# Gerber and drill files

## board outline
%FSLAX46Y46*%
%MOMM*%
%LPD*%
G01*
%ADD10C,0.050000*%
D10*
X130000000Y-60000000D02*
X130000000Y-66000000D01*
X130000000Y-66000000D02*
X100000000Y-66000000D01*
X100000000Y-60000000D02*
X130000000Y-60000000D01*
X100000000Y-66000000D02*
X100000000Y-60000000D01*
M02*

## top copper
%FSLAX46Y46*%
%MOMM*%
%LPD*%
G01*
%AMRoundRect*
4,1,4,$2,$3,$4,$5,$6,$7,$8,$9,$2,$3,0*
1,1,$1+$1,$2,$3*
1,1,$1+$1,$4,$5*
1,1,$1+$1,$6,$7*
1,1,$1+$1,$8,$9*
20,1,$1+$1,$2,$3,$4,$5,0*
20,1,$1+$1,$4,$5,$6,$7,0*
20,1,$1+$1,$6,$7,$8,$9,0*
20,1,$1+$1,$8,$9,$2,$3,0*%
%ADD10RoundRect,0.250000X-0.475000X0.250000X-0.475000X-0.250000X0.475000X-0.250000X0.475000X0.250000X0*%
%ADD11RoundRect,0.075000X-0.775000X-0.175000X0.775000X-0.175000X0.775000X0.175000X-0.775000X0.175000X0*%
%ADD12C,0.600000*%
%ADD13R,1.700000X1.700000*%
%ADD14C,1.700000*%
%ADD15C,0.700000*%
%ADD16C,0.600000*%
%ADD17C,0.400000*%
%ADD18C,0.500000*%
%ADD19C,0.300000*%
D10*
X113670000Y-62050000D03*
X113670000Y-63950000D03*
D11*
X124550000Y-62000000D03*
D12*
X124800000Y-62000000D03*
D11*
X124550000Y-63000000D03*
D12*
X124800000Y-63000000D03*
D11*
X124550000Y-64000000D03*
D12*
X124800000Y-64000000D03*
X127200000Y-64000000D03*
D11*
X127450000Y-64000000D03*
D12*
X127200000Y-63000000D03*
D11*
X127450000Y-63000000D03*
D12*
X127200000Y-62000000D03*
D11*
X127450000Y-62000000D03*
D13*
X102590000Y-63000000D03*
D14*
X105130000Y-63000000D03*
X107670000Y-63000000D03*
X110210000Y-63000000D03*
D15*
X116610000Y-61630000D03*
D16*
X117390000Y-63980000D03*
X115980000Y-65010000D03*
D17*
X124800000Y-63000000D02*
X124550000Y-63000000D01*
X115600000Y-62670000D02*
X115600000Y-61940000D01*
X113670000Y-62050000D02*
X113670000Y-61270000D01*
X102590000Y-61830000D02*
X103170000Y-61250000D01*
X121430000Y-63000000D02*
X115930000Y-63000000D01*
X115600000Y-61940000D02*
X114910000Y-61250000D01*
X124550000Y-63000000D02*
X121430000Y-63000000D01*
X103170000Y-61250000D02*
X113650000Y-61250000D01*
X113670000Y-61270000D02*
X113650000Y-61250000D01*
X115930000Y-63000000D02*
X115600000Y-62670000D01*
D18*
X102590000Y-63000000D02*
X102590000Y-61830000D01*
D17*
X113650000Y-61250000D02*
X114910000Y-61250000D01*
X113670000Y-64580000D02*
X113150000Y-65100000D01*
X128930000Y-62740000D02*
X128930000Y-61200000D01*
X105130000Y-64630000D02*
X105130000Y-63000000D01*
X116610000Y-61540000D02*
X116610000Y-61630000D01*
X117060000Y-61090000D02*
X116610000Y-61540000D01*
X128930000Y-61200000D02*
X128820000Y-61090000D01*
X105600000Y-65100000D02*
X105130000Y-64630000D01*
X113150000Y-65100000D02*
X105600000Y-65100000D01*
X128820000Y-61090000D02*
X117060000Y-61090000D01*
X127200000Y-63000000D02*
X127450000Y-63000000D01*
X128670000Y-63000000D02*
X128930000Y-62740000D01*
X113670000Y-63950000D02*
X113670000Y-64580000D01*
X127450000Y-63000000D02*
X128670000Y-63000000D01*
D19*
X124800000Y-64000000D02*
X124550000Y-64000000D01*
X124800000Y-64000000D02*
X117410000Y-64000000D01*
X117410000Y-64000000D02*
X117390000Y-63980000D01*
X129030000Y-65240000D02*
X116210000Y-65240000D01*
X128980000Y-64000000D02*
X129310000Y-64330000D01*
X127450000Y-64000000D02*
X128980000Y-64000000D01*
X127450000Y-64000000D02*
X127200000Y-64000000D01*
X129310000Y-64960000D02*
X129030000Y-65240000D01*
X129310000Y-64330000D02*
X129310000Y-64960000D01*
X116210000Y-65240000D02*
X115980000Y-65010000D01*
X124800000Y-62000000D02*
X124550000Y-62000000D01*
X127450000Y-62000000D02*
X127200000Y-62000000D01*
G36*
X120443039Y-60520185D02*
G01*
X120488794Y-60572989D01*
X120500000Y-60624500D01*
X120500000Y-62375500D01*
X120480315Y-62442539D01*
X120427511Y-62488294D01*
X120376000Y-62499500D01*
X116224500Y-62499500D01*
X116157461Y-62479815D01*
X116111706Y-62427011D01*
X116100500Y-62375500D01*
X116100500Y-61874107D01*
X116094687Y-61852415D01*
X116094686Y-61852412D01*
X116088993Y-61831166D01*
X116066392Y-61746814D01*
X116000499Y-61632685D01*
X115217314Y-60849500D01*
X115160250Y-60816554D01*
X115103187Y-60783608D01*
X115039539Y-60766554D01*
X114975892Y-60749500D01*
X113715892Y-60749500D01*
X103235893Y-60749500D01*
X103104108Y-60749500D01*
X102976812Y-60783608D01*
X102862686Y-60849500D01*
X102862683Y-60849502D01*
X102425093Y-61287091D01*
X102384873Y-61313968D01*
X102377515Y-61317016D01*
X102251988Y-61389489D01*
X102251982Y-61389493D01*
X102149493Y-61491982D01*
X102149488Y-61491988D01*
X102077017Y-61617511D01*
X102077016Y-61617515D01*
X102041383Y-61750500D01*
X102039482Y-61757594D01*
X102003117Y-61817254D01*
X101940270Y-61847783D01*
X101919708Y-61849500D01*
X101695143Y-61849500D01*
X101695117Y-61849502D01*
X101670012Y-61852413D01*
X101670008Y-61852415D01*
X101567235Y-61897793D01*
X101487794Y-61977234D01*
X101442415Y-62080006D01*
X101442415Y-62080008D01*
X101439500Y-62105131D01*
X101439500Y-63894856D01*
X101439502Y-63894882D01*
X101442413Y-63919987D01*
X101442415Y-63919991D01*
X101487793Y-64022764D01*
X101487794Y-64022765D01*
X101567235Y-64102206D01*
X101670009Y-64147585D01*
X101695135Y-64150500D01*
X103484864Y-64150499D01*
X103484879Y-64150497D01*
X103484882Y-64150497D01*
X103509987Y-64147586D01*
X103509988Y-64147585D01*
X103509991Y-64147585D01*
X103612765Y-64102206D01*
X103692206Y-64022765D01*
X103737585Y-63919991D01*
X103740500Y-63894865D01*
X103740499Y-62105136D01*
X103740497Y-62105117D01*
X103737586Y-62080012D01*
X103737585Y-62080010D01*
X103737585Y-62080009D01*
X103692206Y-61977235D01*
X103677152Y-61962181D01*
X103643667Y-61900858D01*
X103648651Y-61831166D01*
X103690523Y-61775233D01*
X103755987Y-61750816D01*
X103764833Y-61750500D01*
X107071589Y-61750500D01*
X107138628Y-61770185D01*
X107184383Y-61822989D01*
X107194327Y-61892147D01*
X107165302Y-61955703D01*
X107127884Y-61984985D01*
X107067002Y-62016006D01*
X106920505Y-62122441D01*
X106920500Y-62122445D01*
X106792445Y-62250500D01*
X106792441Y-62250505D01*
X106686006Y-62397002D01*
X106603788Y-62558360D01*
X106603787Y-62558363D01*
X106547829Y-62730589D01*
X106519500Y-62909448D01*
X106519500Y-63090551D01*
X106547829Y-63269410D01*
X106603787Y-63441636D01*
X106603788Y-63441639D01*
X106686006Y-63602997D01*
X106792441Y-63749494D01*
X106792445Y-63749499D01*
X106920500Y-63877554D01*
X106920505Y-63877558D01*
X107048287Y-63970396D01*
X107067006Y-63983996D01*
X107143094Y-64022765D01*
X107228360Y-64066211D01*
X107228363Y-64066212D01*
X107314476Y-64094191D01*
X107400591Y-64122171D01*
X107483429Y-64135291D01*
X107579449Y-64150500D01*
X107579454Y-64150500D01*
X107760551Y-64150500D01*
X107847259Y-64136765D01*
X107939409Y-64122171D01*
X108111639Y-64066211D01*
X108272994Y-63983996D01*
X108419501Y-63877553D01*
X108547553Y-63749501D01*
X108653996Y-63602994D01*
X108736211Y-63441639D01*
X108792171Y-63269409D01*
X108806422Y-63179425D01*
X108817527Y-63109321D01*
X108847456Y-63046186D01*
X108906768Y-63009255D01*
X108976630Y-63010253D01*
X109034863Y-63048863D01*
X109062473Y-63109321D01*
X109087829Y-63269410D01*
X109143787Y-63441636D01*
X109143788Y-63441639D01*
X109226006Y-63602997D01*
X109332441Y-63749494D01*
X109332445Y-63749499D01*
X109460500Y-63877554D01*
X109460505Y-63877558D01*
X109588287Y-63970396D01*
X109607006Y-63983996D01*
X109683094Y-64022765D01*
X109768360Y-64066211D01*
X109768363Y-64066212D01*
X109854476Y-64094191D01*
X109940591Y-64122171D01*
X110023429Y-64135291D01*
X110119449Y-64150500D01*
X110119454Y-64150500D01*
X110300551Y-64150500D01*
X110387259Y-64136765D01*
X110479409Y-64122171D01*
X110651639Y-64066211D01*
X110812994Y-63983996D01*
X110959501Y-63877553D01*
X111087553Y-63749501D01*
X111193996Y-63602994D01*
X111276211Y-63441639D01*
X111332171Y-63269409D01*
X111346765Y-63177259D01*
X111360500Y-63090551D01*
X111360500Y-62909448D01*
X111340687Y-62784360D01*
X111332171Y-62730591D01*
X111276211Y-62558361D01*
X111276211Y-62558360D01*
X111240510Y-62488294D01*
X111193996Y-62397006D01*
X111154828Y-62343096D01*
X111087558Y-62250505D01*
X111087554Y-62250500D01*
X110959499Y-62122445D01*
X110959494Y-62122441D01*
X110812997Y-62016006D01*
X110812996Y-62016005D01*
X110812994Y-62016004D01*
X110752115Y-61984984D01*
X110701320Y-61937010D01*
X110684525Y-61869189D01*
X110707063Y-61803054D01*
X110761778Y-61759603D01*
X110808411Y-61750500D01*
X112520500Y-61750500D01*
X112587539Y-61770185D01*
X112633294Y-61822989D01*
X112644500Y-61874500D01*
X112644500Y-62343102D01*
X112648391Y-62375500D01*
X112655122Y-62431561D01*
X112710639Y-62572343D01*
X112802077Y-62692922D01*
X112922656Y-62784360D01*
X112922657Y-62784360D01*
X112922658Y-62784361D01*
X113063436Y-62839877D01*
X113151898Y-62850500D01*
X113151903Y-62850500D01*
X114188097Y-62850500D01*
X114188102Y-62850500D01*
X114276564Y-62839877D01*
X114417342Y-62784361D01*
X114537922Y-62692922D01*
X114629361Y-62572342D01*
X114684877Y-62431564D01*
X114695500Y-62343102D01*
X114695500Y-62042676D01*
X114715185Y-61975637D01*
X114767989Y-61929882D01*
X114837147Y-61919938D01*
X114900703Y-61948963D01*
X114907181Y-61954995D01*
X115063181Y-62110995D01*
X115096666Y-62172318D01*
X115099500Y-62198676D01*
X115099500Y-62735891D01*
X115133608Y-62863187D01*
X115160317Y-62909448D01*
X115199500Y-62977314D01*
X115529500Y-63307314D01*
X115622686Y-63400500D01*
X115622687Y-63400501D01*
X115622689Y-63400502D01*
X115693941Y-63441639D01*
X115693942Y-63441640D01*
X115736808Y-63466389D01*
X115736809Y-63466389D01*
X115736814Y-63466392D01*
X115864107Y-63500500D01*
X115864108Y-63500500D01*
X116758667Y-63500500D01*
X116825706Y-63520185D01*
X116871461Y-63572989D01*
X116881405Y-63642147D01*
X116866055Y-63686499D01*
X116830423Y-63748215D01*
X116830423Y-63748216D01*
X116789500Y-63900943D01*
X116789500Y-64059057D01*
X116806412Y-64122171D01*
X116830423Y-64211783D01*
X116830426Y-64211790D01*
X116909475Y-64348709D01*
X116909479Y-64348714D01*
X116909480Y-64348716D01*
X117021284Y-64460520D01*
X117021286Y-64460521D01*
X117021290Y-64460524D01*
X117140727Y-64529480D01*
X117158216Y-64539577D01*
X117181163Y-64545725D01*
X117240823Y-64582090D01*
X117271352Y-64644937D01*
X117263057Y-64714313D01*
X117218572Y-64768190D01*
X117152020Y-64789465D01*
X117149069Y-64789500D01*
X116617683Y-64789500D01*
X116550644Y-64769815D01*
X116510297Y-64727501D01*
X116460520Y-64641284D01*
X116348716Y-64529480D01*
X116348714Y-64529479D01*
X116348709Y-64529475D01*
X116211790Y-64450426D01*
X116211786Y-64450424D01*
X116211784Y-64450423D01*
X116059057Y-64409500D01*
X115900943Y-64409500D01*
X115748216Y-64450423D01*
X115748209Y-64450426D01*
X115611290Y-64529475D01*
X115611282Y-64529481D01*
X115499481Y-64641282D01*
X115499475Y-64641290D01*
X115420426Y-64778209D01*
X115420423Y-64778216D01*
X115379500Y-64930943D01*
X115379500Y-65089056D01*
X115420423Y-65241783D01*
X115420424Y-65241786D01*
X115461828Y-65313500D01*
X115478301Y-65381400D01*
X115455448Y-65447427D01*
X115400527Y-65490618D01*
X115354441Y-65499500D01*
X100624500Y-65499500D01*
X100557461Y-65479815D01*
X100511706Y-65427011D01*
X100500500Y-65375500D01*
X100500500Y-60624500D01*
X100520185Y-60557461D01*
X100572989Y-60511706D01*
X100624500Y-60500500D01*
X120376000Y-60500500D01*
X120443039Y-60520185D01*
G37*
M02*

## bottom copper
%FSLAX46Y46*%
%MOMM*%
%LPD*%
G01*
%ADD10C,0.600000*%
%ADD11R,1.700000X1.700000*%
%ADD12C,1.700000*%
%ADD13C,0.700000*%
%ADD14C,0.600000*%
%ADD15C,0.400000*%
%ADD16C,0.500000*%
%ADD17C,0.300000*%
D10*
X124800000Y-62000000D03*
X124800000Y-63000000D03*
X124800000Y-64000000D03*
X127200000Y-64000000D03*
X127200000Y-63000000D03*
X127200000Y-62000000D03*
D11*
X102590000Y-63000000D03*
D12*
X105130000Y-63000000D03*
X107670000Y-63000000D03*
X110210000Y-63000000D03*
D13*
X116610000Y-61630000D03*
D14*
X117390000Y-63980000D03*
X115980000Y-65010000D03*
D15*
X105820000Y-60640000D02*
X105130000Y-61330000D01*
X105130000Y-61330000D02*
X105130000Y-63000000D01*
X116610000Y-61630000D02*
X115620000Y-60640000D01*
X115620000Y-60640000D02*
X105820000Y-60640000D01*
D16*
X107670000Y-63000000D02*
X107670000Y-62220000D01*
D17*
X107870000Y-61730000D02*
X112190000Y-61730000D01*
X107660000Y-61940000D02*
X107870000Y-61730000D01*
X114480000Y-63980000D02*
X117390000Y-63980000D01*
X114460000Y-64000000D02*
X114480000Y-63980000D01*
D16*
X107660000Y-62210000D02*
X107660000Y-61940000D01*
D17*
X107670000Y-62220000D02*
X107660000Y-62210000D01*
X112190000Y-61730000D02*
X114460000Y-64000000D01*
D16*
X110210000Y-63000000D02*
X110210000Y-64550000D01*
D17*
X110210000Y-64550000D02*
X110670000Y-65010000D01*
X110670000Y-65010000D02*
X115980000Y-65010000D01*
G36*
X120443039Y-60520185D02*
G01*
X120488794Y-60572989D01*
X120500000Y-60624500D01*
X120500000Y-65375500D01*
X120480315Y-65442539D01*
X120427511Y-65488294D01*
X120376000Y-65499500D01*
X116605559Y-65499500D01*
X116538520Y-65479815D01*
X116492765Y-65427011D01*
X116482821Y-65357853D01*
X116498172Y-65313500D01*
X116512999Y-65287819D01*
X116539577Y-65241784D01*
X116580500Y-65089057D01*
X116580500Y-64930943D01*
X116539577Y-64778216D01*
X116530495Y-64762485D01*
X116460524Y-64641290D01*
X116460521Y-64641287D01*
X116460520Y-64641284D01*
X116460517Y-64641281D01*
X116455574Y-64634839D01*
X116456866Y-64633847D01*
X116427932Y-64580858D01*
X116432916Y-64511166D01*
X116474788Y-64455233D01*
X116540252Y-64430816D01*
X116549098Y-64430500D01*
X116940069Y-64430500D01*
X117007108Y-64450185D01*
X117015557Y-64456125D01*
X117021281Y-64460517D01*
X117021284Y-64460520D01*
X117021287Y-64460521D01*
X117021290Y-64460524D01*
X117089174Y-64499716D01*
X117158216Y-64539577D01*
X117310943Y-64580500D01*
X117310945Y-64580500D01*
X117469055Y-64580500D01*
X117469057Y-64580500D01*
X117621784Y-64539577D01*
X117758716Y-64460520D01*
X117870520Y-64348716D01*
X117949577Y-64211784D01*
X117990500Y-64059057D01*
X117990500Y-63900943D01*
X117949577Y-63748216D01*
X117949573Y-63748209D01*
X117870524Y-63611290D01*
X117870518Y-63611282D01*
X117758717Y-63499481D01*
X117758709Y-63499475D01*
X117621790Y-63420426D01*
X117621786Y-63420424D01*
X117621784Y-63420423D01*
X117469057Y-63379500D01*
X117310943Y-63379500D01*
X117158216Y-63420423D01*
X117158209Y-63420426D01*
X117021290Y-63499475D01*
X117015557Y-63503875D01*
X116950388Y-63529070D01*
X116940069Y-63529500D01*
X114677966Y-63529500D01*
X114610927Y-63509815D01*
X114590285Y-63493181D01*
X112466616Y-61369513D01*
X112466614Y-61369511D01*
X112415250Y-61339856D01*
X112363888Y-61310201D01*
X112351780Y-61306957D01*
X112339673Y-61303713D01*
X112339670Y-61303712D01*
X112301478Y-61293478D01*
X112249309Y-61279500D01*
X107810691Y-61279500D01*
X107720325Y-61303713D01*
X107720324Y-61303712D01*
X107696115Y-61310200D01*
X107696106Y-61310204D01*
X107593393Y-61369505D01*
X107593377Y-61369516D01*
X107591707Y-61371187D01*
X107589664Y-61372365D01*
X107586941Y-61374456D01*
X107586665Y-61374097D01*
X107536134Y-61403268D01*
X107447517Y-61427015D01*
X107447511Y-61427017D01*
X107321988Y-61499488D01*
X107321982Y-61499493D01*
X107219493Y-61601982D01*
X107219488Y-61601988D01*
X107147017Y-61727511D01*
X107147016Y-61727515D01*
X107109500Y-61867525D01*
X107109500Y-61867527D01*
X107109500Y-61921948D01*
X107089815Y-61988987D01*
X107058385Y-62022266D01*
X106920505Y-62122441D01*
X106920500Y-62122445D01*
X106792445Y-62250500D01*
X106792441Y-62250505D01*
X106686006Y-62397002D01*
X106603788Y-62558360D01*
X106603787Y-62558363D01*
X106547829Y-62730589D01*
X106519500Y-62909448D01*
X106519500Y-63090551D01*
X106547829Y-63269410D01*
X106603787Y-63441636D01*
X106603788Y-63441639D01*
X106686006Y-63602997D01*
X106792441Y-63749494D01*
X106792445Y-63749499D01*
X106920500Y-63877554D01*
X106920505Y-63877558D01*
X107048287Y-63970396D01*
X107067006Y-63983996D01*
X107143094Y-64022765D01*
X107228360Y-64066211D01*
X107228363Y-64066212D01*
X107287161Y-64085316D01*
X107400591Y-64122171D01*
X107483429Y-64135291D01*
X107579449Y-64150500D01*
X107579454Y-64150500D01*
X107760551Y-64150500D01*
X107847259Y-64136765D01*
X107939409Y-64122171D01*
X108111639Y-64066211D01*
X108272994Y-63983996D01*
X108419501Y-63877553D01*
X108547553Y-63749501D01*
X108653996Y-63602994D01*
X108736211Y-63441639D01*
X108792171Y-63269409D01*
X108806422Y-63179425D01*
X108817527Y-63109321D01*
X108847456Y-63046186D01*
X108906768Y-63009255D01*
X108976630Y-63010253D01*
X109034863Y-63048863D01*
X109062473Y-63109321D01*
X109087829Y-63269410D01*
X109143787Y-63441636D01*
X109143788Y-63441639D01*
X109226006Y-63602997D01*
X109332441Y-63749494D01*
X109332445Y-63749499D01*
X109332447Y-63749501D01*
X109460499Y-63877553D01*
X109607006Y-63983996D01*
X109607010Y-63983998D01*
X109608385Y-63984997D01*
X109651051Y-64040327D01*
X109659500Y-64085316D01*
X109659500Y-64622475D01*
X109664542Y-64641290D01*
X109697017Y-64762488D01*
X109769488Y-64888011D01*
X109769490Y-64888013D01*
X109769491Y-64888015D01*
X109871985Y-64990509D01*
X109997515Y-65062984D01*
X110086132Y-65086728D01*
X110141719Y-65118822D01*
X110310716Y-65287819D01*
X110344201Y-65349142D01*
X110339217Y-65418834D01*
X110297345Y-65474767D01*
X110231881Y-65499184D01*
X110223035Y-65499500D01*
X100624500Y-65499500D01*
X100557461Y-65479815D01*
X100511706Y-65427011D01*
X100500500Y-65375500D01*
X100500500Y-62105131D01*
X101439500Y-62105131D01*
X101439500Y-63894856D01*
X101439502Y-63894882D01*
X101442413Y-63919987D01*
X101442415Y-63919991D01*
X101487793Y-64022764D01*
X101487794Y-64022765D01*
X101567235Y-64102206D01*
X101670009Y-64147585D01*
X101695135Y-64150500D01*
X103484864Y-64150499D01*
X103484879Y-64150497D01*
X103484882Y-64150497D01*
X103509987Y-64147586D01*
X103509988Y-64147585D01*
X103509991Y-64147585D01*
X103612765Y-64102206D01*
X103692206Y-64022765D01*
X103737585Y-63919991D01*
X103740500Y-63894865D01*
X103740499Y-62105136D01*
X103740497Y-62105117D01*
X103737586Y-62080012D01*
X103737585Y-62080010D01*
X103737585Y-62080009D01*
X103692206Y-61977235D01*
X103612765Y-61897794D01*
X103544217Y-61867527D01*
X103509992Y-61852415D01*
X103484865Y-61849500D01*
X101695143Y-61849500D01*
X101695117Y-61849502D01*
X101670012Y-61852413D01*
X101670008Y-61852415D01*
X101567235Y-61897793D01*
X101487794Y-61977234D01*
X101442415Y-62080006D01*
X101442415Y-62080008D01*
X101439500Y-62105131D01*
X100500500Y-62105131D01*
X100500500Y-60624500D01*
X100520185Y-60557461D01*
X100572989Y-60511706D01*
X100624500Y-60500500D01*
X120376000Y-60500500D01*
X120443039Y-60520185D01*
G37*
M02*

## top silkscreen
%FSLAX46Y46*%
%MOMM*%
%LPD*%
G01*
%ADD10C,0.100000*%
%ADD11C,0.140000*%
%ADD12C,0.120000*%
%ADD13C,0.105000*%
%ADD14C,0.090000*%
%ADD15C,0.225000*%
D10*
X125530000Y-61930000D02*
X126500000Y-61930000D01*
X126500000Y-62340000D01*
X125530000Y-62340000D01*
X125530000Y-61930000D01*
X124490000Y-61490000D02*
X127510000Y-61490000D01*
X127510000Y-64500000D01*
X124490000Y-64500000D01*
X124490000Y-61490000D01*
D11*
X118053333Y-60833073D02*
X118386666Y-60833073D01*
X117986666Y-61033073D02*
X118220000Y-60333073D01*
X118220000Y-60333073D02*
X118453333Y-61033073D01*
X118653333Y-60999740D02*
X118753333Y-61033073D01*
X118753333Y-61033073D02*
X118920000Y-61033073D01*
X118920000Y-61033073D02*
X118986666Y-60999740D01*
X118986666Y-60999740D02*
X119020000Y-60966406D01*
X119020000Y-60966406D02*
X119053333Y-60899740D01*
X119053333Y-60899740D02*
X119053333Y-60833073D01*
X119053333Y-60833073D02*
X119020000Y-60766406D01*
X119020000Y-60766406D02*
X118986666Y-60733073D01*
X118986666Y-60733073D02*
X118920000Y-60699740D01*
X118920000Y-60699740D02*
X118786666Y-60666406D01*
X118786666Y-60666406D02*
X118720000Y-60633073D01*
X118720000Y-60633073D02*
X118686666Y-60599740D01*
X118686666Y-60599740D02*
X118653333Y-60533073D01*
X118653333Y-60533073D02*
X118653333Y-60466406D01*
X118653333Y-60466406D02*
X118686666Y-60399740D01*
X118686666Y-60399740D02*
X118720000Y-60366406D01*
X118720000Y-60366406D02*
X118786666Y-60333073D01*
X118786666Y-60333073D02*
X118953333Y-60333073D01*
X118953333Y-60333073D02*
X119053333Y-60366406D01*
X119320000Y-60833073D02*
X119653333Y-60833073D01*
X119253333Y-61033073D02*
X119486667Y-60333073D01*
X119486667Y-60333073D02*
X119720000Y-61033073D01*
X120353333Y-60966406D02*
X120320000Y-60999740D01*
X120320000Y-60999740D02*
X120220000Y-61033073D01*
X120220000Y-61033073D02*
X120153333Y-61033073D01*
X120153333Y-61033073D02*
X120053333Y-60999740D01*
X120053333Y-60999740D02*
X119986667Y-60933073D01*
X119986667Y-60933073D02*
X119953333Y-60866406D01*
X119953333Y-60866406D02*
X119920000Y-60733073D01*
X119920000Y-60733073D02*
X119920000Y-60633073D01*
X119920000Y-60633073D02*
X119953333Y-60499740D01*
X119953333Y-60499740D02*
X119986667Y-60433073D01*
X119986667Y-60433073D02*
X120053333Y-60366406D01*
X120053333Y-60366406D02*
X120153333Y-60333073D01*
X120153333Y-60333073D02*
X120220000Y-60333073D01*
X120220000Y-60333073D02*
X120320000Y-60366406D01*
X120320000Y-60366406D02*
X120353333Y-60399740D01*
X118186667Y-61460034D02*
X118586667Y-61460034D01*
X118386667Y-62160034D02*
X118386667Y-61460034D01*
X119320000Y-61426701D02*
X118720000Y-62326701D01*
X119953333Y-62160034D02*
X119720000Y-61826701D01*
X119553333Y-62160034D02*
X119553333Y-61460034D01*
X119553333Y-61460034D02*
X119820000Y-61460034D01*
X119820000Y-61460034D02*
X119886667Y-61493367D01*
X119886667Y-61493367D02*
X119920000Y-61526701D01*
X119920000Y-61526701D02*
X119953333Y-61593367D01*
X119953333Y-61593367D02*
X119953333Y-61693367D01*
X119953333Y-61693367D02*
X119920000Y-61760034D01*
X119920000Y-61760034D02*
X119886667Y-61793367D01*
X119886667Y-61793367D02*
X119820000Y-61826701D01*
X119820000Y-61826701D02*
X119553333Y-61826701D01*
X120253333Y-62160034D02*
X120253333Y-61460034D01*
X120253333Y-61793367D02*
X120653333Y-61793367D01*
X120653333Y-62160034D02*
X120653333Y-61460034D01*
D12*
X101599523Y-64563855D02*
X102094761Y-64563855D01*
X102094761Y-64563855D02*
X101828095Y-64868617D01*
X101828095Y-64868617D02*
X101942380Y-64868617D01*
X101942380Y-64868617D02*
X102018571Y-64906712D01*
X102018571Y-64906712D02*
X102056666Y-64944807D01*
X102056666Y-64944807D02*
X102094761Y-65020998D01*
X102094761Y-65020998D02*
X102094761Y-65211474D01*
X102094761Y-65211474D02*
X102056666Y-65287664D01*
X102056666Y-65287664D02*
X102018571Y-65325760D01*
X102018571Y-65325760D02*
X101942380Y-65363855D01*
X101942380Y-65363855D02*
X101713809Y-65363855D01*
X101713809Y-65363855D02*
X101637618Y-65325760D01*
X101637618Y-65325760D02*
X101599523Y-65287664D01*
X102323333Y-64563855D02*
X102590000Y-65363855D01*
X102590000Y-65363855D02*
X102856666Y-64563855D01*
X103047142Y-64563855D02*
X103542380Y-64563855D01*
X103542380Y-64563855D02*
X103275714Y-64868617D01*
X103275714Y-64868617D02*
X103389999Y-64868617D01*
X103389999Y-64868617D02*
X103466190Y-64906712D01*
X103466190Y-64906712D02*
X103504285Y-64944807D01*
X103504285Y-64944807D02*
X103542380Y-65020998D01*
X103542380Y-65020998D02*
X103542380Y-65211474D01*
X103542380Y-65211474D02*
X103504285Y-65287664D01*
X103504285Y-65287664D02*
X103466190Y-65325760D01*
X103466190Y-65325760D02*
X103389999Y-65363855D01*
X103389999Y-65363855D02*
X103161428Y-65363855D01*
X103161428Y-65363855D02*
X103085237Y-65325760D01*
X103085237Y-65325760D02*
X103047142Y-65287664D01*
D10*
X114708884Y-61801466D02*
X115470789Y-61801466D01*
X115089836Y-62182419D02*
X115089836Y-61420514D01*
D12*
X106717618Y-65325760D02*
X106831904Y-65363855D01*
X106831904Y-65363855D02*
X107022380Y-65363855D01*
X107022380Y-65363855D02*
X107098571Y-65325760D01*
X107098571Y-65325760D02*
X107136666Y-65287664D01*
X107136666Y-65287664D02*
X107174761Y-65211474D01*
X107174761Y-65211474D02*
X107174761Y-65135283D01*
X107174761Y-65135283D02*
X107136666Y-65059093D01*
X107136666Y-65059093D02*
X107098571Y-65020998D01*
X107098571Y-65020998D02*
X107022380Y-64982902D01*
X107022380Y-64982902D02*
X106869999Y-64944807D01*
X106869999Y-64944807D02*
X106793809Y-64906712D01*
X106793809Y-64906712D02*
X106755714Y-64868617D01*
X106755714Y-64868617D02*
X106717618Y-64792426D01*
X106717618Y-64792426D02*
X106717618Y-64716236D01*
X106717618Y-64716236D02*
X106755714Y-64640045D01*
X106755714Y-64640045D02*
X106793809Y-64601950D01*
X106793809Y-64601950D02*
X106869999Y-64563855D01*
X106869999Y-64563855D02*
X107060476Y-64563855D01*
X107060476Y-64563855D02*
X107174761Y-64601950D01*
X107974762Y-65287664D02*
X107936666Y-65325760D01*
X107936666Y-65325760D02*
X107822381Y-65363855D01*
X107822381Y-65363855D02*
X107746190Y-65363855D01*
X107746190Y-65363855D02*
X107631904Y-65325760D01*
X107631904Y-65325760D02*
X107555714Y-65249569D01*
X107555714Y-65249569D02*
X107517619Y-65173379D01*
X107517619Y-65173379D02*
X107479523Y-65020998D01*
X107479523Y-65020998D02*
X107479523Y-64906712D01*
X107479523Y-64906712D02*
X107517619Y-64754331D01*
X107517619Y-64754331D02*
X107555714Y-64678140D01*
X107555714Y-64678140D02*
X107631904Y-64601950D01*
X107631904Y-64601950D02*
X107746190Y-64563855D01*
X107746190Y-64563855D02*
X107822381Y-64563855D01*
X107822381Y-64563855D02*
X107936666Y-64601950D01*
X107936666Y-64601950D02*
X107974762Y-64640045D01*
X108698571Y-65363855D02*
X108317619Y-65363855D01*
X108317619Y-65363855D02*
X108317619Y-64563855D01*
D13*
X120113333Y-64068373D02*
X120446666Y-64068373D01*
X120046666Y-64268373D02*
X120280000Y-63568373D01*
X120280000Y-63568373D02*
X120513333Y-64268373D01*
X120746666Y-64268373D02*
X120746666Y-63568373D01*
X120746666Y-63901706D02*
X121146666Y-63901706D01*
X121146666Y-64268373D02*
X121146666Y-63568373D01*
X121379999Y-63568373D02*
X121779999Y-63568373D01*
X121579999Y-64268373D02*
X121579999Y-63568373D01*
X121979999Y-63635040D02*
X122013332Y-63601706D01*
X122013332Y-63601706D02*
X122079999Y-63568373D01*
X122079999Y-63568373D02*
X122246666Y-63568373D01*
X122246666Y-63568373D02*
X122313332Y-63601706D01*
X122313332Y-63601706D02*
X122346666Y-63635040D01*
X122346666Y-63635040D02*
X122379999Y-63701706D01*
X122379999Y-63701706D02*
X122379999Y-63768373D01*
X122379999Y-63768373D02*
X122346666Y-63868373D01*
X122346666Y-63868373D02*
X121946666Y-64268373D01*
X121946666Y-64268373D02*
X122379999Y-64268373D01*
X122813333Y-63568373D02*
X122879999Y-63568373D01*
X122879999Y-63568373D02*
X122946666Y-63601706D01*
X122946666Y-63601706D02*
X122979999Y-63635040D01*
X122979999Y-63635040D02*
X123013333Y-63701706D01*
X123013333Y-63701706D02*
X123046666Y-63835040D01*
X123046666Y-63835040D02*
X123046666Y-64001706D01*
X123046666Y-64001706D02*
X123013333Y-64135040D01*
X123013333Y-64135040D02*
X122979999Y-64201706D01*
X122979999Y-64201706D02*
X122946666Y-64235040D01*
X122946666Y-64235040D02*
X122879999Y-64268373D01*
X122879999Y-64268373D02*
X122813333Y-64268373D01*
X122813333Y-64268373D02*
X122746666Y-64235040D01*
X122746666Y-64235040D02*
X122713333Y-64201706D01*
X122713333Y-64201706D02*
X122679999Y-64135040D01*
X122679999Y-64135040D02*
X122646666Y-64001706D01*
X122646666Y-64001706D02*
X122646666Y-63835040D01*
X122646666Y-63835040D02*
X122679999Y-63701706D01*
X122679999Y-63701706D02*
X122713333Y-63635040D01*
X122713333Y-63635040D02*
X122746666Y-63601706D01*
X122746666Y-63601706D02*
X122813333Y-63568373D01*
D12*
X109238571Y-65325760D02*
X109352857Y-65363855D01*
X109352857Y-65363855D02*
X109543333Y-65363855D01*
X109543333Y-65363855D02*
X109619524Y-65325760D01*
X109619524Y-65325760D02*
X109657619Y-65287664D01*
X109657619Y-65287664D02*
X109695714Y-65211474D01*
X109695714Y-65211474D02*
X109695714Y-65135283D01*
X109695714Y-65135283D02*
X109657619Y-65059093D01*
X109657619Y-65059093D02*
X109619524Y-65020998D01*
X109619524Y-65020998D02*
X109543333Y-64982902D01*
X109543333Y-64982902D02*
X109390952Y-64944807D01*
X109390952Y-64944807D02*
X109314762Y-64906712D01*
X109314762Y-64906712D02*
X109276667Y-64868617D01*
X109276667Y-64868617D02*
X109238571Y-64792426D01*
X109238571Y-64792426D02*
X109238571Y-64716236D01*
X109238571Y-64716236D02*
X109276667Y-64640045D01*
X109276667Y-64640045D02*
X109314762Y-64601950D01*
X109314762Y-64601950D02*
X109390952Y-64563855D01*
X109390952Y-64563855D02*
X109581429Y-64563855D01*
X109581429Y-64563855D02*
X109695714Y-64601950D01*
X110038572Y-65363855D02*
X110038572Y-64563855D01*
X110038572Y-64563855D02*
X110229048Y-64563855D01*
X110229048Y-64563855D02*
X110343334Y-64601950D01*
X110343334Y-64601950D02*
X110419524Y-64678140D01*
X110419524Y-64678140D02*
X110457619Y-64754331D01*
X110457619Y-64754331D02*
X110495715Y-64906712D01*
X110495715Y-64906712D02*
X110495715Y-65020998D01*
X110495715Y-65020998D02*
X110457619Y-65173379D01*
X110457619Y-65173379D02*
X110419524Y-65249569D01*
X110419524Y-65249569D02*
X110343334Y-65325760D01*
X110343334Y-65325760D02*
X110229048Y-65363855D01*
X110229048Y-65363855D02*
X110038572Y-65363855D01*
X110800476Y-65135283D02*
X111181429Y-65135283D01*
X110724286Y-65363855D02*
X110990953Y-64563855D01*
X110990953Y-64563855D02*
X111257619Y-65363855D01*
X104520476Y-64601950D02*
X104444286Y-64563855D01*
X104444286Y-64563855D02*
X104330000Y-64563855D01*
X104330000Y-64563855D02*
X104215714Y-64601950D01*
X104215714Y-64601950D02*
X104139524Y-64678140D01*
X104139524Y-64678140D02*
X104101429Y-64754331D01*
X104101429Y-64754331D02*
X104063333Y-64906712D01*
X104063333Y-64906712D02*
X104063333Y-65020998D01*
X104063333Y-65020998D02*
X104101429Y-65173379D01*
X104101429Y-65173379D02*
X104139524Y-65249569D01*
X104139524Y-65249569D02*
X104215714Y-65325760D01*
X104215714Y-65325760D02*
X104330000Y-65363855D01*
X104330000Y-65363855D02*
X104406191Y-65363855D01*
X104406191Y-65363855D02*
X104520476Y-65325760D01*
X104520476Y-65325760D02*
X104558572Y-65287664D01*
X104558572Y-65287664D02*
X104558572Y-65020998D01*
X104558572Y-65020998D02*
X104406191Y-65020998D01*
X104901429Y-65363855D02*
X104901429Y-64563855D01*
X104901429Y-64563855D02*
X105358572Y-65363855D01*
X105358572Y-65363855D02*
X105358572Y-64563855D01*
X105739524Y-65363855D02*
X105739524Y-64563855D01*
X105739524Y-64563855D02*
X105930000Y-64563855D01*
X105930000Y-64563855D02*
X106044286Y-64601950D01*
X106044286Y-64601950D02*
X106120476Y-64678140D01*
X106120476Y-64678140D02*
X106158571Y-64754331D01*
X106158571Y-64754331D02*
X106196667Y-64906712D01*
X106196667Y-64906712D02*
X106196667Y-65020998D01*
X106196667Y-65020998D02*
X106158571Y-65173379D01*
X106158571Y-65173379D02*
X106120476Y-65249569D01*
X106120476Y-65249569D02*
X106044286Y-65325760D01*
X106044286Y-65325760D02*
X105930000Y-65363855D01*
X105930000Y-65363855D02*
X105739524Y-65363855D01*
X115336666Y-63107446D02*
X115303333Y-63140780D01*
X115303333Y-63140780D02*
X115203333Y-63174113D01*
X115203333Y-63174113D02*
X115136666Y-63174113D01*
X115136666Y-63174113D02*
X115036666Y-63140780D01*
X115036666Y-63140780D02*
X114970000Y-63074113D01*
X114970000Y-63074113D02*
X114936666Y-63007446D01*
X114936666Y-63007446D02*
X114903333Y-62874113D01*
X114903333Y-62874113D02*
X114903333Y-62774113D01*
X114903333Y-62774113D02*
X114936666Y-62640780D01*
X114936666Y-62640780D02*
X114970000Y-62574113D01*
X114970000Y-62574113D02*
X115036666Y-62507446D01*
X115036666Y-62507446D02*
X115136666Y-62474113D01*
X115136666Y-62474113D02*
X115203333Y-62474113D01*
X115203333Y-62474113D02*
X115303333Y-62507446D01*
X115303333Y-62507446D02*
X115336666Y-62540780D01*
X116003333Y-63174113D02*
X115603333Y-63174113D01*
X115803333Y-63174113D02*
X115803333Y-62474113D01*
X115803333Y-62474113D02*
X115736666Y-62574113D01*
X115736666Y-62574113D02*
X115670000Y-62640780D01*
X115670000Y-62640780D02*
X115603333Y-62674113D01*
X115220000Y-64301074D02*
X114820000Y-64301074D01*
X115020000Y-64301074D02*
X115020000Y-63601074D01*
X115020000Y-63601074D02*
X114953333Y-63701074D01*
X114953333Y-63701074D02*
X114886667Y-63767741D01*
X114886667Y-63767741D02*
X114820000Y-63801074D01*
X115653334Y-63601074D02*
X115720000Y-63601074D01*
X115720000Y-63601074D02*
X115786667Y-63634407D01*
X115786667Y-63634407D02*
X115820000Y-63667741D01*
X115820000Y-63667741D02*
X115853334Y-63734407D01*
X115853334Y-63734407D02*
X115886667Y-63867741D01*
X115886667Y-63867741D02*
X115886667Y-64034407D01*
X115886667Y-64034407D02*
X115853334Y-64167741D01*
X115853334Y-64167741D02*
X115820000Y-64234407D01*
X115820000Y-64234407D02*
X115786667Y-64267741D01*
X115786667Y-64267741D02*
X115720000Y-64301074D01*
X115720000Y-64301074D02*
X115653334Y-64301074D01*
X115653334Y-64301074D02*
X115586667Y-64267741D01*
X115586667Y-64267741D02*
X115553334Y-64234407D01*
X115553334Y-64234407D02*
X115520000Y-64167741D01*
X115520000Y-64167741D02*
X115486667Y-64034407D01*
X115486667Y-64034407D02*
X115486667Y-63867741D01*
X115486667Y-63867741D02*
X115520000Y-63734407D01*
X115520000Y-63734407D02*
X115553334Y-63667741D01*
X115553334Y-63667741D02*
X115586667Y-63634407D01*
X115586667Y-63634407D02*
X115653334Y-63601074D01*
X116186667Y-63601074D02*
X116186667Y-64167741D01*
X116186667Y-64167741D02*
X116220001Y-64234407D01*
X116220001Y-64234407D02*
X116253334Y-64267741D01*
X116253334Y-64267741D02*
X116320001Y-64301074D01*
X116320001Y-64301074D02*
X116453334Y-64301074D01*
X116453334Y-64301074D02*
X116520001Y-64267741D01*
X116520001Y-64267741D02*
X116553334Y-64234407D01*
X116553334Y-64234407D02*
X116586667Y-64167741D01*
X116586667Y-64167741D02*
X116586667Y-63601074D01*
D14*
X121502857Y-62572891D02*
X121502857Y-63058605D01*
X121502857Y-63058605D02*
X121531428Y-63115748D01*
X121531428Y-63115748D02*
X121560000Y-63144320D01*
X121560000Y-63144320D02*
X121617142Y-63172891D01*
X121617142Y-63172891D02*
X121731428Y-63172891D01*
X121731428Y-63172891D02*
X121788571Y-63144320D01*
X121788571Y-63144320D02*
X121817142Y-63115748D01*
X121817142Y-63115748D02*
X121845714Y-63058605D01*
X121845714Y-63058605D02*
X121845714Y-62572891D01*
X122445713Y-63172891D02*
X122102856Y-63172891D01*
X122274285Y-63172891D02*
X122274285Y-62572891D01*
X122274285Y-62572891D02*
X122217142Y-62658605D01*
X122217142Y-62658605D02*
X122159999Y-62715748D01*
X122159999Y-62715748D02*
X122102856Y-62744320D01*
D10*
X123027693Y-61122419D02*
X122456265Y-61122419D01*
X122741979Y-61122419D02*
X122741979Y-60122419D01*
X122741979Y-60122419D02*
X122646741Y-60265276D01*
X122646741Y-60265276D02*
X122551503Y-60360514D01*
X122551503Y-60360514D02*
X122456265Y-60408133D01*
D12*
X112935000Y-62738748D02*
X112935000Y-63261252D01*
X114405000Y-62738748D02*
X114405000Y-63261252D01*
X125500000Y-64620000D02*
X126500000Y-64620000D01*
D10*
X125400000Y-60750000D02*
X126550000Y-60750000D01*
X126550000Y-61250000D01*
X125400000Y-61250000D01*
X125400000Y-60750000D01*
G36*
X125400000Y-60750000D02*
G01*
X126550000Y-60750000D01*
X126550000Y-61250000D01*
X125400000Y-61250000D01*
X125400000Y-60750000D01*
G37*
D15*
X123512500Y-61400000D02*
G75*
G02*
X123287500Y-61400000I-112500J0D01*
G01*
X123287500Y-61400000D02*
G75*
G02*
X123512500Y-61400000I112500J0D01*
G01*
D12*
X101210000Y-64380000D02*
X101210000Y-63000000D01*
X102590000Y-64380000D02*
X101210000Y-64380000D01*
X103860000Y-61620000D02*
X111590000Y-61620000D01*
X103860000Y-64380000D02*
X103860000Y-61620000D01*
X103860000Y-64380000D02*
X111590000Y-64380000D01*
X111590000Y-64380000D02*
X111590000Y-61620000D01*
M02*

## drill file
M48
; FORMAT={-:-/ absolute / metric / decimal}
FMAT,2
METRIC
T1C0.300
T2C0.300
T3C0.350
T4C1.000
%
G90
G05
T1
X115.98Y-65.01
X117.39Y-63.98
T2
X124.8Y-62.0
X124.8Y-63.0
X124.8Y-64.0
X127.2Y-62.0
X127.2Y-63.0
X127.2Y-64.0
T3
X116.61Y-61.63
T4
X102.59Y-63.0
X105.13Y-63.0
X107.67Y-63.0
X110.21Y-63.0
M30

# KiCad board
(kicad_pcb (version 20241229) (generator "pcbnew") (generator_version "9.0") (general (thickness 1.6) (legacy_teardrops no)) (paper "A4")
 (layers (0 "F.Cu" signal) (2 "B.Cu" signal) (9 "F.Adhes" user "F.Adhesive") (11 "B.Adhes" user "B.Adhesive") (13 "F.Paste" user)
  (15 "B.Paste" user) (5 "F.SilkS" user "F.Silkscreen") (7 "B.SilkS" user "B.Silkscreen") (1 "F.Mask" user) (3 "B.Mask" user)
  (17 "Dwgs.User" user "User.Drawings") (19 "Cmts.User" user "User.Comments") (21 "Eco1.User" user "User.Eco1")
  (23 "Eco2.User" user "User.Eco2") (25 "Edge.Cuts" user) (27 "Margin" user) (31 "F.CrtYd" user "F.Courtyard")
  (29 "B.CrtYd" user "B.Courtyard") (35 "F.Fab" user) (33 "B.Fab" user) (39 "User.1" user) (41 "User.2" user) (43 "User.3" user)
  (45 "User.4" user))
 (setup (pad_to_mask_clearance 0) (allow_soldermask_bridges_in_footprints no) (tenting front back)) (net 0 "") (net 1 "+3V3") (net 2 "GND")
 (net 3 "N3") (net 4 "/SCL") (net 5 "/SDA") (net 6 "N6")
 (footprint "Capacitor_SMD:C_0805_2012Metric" (layer "F.Cu") (at 113.67 63 -90)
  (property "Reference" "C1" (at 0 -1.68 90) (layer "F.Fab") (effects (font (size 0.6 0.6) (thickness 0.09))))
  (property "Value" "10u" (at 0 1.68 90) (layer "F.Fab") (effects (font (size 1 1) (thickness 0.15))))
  (fp_line (start -0.261252 0.735) (end 0.261252 0.735) (stroke (width 0.12) (type solid)) (layer "F.SilkS"))
  (fp_line (start -0.261252 -0.735) (end 0.261252 -0.735) (stroke (width 0.12) (type solid)) (layer "F.SilkS"))
  (pad "1" smd roundrect (at -0.95 0 270) (size 1 1.45) (layers "F.Cu" "F.Mask" "F.Paste") (roundrect_rratio 0.25) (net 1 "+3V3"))
  (pad "2" smd roundrect (at 0.95 0 270) (size 1 1.45) (layers "F.Cu" "F.Mask" "F.Paste") (roundrect_rratio 0.25) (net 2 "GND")))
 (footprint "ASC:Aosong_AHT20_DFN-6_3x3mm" (layer "F.Cu") (at 126 63)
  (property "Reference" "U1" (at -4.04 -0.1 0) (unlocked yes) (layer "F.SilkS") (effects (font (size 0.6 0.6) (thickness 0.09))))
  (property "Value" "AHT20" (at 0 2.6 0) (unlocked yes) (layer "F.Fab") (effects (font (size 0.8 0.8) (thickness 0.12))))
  (fp_line (start -0.5 1.62) (end 0.5 1.62) (stroke (width 0.12) (type solid)) (layer "F.SilkS"))
  (fp_rect (start -0.6 -2.25) (end 0.55 -1.75) (stroke (width 0.1) (type solid)) (fill yes) (layer "F.SilkS"))
  (fp_circle (center -2.6 -1.6) (end -2.45 -1.6) (stroke (width 0.15) (type solid)) (fill yes) (layer "F.SilkS"))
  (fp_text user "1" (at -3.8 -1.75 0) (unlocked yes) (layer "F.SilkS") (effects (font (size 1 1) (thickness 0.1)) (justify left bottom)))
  (pad "1" smd roundrect (at -1.45 -1) (size 1.7 0.5) (layers "F.Cu" "F.Mask" "F.Paste") (roundrect_rratio 0.15) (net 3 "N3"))
  (pad "1" thru_hole circle (at -1.2 -1) (size 0.6 0.6) (drill 0.3) (layers "*.Cu" "*.Mask") (remove_unused_layers no) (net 3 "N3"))
  (pad "2" smd roundrect (at -1.45 0) (size 1.7 0.5) (layers "F.Cu" "F.Mask" "F.Paste") (roundrect_rratio 0.15) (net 1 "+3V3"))
  (pad "2" thru_hole circle (at -1.2 0) (size 0.6 0.6) (drill 0.3) (layers "*.Cu" "*.Mask") (remove_unused_layers no) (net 1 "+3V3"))
  (pad "3" smd roundrect (at -1.45 1) (size 1.7 0.5) (layers "F.Cu" "F.Mask" "F.Paste") (roundrect_rratio 0.15) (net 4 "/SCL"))
  (pad "3" thru_hole circle (at -1.2 1) (size 0.6 0.6) (drill 0.3) (layers "*.Cu" "*.Mask") (remove_unused_layers no) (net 4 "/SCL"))
  (pad "4" thru_hole circle (at 1.2 1) (size 0.6 0.6) (drill 0.3) (layers "*.Cu" "*.Mask") (remove_unused_layers no) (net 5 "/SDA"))
  (pad "4" smd roundrect (at 1.45 1) (size 1.7 0.5) (layers "F.Cu" "F.Mask" "F.Paste") (roundrect_rratio 0.15) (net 5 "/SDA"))
  (pad "5" thru_hole circle (at 1.2 0) (size 0.6 0.6) (drill 0.3) (layers "*.Cu" "*.Mask") (remove_unused_layers no) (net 2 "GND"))
  (pad "5" smd roundrect (at 1.45 0) (size 1.7 0.5) (layers "F.Cu" "F.Mask" "F.Paste") (roundrect_rratio 0.15) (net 2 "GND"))
  (pad "6" thru_hole circle (at 1.2 -1) (size 0.6 0.6) (drill 0.3) (layers "*.Cu" "*.Mask") (remove_unused_layers no) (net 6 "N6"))
  (pad "6" smd roundrect (at 1.45 -1) (size 1.7 0.5) (layers "F.Cu" "F.Mask" "F.Paste") (roundrect_rratio 0.15) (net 6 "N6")))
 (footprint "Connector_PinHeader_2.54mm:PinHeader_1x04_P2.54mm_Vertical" (layer "F.Cu") (at 102.59 63 90)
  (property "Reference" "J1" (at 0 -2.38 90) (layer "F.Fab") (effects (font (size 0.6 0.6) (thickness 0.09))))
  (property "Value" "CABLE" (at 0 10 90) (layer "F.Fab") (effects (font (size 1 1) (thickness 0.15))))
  (fp_line (start -1.38 -1.38) (end 0 -1.38) (stroke (width 0.12) (type solid)) (layer "F.SilkS"))
  (fp_line (start -1.38 0) (end -1.38 -1.38) (stroke (width 0.12) (type solid)) (layer "F.SilkS"))
  (fp_line (start 1.38 1.27) (end 1.38 9) (stroke (width 0.12) (type solid)) (layer "F.SilkS"))
  (fp_line (start -1.38 1.27) (end 1.38 1.27) (stroke (width 0.12) (type solid)) (layer "F.SilkS"))
  (fp_line (start -1.38 1.27) (end -1.38 9) (stroke (width 0.12) (type solid)) (layer "F.SilkS"))
  (fp_line (start -1.38 9) (end 1.38 9) (stroke (width 0.12) (type solid)) (layer "F.SilkS"))
  (pad "1" thru_hole rect (at 0 0 90) (size 1.7 1.7) (drill 1) (layers "*.Cu" "*.Mask") (remove_unused_layers no) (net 1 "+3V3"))
  (pad "2" thru_hole circle (at 0 2.54 90) (size 1.7 1.7) (drill 1) (layers "*.Cu" "*.Mask") (remove_unused_layers no) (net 2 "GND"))
  (pad "3" thru_hole circle (at 0 5.08 90) (size 1.7 1.7) (drill 1) (layers "*.Cu" "*.Mask") (remove_unused_layers no) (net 4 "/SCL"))
  (pad "4" thru_hole circle (at 0 7.62 90) (size 1.7 1.7) (drill 1) (layers "*.Cu" "*.Mask") (remove_unused_layers no) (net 5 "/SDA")))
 (gr_rect (start 125.53 61.93) (end 126.5 62.34) (stroke (width 0.1) (type default)) (fill no) (layer "F.SilkS"))
 (gr_rect (start 124.49 61.49) (end 127.51 64.5) (stroke (width 0.1) (type default)) (fill no) (layer "F.SilkS"))
 (gr_line (start 130 60) (end 130 66) (stroke (width 0.05) (type default)) (layer "Edge.Cuts"))
 (gr_line (start 130 66) (end 100 66) (stroke (width 0.05) (type default)) (layer "Edge.Cuts"))
 (gr_line (start 100 60) (end 130 60) (stroke (width 0.05) (type default)) (layer "Edge.Cuts"))
 (gr_line (start 100 66) (end 100 60) (stroke (width 0.05) (type default)) (layer "Edge.Cuts"))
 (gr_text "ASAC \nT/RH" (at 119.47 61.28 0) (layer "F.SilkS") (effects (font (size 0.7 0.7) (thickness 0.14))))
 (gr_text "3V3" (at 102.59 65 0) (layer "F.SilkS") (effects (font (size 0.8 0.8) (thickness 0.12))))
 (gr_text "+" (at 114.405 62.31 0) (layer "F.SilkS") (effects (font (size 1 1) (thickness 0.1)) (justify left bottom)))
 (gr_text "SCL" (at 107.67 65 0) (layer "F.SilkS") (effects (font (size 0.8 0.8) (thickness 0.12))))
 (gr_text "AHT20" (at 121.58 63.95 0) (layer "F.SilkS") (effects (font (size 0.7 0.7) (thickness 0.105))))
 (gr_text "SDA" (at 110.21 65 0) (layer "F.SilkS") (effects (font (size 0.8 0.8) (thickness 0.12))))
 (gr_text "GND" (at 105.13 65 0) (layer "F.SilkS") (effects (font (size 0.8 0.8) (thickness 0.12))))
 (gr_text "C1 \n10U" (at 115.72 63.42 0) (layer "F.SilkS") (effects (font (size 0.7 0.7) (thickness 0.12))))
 (segment (start 124.8 63) (end 124.55 63) (width 0.4) (layer "F.Cu") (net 1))
 (segment (start 115.6 62.67) (end 115.6 61.94) (width 0.4) (layer "F.Cu") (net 1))
 (segment (start 113.67 62.05) (end 113.67 61.27) (width 0.4) (layer "F.Cu") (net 1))
 (segment (start 102.59 61.83) (end 103.17 61.25) (width 0.4) (layer "F.Cu") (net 1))
 (segment (start 121.43 63) (end 115.93 63) (width 0.4) (layer "F.Cu") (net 1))
 (segment (start 115.6 61.94) (end 114.91 61.25) (width 0.4) (layer "F.Cu") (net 1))
 (segment (start 124.55 63) (end 121.43 63) (width 0.4) (layer "F.Cu") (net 1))
 (segment (start 103.17 61.25) (end 113.65 61.25) (width 0.4) (layer "F.Cu") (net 1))
 (segment (start 113.67 61.27) (end 113.65 61.25) (width 0.4) (layer "F.Cu") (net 1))
 (segment (start 115.93 63) (end 115.6 62.67) (width 0.4) (layer "F.Cu") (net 1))
 (segment (start 102.59 63) (end 102.59 61.83) (width 0.5) (layer "F.Cu") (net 1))
 (segment (start 113.65 61.25) (end 114.91 61.25) (width 0.4) (layer "F.Cu") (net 1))
 (segment (start 113.67 64.58) (end 113.15 65.1) (width 0.4) (layer "F.Cu") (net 2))
 (segment (start 128.93 62.74) (end 128.93 61.2) (width 0.4) (layer "F.Cu") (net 2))
 (segment (start 105.13 64.63) (end 105.13 63) (width 0.4) (layer "F.Cu") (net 2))
 (segment (start 116.61 61.54) (end 116.61 61.63) (width 0.4) (layer "F.Cu") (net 2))
 (segment (start 117.06 61.09) (end 116.61 61.54) (width 0.4) (layer "F.Cu") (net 2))
 (segment (start 128.93 61.2) (end 128.82 61.09) (width 0.4) (layer "F.Cu") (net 2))
 (segment (start 105.6 65.1) (end 105.13 64.63) (width 0.4) (layer "F.Cu") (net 2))
 (segment (start 113.15 65.1) (end 105.6 65.1) (width 0.4) (layer "F.Cu") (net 2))
 (segment (start 128.82 61.09) (end 117.06 61.09) (width 0.4) (layer "F.Cu") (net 2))
 (segment (start 127.2 63) (end 127.45 63) (width 0.4) (layer "F.Cu") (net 2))
 (segment (start 128.67 63) (end 128.93 62.74) (width 0.4) (layer "F.Cu") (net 2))
 (segment (start 113.67 63.95) (end 113.67 64.58) (width 0.4) (layer "F.Cu") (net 2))
 (segment (start 127.45 63) (end 128.67 63) (width 0.4) (layer "F.Cu") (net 2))
 (via (at 116.61 61.63) (size 0.7) (drill 0.35) (layers "F.Cu" "B.Cu") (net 2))
 (segment (start 105.82 60.64) (end 105.13 61.33) (width 0.4) (layer "B.Cu") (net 2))
 (segment (start 105.13 61.33) (end 105.13 63) (width 0.4) (layer "B.Cu") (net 2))
 (segment (start 116.61 61.63) (end 115.62 60.64) (width 0.4) (layer "B.Cu") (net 2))
 (segment (start 115.62 60.64) (end 105.82 60.64) (width 0.4) (layer "B.Cu") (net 2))
 (segment (start 124.8 64) (end 124.55 64) (width 0.3) (layer "F.Cu") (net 4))
 (segment (start 124.8 64) (end 117.41 64) (width 0.3) (layer "F.Cu") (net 4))
 (segment (start 117.41 64) (end 117.39 63.98) (width 0.3) (layer "F.Cu") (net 4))
 (via (at 117.39 63.98) (size 0.6) (drill 0.3) (layers "F.Cu" "B.Cu") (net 4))
 (segment (start 107.67 63) (end 107.67 62.22) (width 0.5) (layer "B.Cu") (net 4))
 (segment (start 107.87 61.73) (end 112.19 61.73) (width 0.3) (layer "B.Cu") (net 4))
 (segment (start 107.66 61.94) (end 107.87 61.73) (width 0.3) (layer "B.Cu") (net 4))
 (segment (start 114.48 63.98) (end 117.39 63.98) (width 0.3) (layer "B.Cu") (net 4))
 (segment (start 114.46 64) (end 114.48 63.98) (width 0.3) (layer "B.Cu") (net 4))
 (segment (start 107.66 62.21) (end 107.66 61.94) (width 0.5) (layer "B.Cu") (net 4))
 (segment (start 107.67 62.22) (end 107.66 62.21) (width 0.3) (layer "B.Cu") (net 4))
 (segment (start 112.19 61.73) (end 114.46 64) (width 0.3) (layer "B.Cu") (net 4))
 (segment (start 129.03 65.24) (end 116.21 65.24) (width 0.3) (layer "F.Cu") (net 5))
 (segment (start 128.98 64) (end 129.31 64.33) (width 0.3) (layer "F.Cu") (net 5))
 (segment (start 127.45 64) (end 128.98 64) (width 0.3) (layer "F.Cu") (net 5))
 (segment (start 127.45 64) (end 127.2 64) (width 0.3) (layer "F.Cu") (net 5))
 (segment (start 129.31 64.96) (end 129.03 65.24) (width 0.3) (layer "F.Cu") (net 5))
 (segment (start 129.31 64.33) (end 129.31 64.96) (width 0.3) (layer "F.Cu") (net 5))
 (segment (start 116.21 65.24) (end 115.98 65.01) (width 0.3) (layer "F.Cu") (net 5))
 (via (at 115.98 65.01) (size 0.6) (drill 0.3) (layers "F.Cu" "B.Cu") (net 5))
 (segment (start 110.21 63) (end 110.21 64.55) (width 0.5) (layer "B.Cu") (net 5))
 (segment (start 110.21 64.55) (end 110.67 65.01) (width 0.3) (layer "B.Cu") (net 5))
 (segment (start 110.67 65.01) (end 115.98 65.01) (width 0.3) (layer "B.Cu") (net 5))
 (segment (start 124.8 62) (end 124.55 62) (width 0.3) (layer "F.Cu") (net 3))
 (segment (start 127.45 62) (end 127.2 62) (width 0.3) (layer "F.Cu") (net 6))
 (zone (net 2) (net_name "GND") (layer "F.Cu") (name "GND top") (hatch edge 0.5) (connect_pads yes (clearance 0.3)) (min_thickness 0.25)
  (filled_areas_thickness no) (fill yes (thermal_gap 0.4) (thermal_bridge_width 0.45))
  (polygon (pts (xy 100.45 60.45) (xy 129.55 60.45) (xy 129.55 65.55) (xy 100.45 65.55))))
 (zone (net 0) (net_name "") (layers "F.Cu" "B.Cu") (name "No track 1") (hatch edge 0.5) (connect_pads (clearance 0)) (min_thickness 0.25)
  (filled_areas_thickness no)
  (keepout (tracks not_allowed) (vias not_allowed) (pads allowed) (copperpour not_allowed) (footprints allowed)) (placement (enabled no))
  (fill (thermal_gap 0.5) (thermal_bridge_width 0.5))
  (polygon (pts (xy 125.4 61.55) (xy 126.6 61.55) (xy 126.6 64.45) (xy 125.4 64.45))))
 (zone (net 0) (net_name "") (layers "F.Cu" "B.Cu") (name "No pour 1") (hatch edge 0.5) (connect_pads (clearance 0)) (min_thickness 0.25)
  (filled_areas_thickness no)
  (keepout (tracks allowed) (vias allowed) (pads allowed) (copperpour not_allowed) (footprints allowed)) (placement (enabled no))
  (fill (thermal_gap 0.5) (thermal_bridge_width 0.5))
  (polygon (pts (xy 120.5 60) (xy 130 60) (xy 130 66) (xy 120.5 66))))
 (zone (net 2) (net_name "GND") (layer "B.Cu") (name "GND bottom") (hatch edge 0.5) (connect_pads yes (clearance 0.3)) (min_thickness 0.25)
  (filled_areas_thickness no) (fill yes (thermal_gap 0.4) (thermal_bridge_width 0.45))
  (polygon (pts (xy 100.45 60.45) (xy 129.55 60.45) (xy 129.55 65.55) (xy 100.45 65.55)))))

